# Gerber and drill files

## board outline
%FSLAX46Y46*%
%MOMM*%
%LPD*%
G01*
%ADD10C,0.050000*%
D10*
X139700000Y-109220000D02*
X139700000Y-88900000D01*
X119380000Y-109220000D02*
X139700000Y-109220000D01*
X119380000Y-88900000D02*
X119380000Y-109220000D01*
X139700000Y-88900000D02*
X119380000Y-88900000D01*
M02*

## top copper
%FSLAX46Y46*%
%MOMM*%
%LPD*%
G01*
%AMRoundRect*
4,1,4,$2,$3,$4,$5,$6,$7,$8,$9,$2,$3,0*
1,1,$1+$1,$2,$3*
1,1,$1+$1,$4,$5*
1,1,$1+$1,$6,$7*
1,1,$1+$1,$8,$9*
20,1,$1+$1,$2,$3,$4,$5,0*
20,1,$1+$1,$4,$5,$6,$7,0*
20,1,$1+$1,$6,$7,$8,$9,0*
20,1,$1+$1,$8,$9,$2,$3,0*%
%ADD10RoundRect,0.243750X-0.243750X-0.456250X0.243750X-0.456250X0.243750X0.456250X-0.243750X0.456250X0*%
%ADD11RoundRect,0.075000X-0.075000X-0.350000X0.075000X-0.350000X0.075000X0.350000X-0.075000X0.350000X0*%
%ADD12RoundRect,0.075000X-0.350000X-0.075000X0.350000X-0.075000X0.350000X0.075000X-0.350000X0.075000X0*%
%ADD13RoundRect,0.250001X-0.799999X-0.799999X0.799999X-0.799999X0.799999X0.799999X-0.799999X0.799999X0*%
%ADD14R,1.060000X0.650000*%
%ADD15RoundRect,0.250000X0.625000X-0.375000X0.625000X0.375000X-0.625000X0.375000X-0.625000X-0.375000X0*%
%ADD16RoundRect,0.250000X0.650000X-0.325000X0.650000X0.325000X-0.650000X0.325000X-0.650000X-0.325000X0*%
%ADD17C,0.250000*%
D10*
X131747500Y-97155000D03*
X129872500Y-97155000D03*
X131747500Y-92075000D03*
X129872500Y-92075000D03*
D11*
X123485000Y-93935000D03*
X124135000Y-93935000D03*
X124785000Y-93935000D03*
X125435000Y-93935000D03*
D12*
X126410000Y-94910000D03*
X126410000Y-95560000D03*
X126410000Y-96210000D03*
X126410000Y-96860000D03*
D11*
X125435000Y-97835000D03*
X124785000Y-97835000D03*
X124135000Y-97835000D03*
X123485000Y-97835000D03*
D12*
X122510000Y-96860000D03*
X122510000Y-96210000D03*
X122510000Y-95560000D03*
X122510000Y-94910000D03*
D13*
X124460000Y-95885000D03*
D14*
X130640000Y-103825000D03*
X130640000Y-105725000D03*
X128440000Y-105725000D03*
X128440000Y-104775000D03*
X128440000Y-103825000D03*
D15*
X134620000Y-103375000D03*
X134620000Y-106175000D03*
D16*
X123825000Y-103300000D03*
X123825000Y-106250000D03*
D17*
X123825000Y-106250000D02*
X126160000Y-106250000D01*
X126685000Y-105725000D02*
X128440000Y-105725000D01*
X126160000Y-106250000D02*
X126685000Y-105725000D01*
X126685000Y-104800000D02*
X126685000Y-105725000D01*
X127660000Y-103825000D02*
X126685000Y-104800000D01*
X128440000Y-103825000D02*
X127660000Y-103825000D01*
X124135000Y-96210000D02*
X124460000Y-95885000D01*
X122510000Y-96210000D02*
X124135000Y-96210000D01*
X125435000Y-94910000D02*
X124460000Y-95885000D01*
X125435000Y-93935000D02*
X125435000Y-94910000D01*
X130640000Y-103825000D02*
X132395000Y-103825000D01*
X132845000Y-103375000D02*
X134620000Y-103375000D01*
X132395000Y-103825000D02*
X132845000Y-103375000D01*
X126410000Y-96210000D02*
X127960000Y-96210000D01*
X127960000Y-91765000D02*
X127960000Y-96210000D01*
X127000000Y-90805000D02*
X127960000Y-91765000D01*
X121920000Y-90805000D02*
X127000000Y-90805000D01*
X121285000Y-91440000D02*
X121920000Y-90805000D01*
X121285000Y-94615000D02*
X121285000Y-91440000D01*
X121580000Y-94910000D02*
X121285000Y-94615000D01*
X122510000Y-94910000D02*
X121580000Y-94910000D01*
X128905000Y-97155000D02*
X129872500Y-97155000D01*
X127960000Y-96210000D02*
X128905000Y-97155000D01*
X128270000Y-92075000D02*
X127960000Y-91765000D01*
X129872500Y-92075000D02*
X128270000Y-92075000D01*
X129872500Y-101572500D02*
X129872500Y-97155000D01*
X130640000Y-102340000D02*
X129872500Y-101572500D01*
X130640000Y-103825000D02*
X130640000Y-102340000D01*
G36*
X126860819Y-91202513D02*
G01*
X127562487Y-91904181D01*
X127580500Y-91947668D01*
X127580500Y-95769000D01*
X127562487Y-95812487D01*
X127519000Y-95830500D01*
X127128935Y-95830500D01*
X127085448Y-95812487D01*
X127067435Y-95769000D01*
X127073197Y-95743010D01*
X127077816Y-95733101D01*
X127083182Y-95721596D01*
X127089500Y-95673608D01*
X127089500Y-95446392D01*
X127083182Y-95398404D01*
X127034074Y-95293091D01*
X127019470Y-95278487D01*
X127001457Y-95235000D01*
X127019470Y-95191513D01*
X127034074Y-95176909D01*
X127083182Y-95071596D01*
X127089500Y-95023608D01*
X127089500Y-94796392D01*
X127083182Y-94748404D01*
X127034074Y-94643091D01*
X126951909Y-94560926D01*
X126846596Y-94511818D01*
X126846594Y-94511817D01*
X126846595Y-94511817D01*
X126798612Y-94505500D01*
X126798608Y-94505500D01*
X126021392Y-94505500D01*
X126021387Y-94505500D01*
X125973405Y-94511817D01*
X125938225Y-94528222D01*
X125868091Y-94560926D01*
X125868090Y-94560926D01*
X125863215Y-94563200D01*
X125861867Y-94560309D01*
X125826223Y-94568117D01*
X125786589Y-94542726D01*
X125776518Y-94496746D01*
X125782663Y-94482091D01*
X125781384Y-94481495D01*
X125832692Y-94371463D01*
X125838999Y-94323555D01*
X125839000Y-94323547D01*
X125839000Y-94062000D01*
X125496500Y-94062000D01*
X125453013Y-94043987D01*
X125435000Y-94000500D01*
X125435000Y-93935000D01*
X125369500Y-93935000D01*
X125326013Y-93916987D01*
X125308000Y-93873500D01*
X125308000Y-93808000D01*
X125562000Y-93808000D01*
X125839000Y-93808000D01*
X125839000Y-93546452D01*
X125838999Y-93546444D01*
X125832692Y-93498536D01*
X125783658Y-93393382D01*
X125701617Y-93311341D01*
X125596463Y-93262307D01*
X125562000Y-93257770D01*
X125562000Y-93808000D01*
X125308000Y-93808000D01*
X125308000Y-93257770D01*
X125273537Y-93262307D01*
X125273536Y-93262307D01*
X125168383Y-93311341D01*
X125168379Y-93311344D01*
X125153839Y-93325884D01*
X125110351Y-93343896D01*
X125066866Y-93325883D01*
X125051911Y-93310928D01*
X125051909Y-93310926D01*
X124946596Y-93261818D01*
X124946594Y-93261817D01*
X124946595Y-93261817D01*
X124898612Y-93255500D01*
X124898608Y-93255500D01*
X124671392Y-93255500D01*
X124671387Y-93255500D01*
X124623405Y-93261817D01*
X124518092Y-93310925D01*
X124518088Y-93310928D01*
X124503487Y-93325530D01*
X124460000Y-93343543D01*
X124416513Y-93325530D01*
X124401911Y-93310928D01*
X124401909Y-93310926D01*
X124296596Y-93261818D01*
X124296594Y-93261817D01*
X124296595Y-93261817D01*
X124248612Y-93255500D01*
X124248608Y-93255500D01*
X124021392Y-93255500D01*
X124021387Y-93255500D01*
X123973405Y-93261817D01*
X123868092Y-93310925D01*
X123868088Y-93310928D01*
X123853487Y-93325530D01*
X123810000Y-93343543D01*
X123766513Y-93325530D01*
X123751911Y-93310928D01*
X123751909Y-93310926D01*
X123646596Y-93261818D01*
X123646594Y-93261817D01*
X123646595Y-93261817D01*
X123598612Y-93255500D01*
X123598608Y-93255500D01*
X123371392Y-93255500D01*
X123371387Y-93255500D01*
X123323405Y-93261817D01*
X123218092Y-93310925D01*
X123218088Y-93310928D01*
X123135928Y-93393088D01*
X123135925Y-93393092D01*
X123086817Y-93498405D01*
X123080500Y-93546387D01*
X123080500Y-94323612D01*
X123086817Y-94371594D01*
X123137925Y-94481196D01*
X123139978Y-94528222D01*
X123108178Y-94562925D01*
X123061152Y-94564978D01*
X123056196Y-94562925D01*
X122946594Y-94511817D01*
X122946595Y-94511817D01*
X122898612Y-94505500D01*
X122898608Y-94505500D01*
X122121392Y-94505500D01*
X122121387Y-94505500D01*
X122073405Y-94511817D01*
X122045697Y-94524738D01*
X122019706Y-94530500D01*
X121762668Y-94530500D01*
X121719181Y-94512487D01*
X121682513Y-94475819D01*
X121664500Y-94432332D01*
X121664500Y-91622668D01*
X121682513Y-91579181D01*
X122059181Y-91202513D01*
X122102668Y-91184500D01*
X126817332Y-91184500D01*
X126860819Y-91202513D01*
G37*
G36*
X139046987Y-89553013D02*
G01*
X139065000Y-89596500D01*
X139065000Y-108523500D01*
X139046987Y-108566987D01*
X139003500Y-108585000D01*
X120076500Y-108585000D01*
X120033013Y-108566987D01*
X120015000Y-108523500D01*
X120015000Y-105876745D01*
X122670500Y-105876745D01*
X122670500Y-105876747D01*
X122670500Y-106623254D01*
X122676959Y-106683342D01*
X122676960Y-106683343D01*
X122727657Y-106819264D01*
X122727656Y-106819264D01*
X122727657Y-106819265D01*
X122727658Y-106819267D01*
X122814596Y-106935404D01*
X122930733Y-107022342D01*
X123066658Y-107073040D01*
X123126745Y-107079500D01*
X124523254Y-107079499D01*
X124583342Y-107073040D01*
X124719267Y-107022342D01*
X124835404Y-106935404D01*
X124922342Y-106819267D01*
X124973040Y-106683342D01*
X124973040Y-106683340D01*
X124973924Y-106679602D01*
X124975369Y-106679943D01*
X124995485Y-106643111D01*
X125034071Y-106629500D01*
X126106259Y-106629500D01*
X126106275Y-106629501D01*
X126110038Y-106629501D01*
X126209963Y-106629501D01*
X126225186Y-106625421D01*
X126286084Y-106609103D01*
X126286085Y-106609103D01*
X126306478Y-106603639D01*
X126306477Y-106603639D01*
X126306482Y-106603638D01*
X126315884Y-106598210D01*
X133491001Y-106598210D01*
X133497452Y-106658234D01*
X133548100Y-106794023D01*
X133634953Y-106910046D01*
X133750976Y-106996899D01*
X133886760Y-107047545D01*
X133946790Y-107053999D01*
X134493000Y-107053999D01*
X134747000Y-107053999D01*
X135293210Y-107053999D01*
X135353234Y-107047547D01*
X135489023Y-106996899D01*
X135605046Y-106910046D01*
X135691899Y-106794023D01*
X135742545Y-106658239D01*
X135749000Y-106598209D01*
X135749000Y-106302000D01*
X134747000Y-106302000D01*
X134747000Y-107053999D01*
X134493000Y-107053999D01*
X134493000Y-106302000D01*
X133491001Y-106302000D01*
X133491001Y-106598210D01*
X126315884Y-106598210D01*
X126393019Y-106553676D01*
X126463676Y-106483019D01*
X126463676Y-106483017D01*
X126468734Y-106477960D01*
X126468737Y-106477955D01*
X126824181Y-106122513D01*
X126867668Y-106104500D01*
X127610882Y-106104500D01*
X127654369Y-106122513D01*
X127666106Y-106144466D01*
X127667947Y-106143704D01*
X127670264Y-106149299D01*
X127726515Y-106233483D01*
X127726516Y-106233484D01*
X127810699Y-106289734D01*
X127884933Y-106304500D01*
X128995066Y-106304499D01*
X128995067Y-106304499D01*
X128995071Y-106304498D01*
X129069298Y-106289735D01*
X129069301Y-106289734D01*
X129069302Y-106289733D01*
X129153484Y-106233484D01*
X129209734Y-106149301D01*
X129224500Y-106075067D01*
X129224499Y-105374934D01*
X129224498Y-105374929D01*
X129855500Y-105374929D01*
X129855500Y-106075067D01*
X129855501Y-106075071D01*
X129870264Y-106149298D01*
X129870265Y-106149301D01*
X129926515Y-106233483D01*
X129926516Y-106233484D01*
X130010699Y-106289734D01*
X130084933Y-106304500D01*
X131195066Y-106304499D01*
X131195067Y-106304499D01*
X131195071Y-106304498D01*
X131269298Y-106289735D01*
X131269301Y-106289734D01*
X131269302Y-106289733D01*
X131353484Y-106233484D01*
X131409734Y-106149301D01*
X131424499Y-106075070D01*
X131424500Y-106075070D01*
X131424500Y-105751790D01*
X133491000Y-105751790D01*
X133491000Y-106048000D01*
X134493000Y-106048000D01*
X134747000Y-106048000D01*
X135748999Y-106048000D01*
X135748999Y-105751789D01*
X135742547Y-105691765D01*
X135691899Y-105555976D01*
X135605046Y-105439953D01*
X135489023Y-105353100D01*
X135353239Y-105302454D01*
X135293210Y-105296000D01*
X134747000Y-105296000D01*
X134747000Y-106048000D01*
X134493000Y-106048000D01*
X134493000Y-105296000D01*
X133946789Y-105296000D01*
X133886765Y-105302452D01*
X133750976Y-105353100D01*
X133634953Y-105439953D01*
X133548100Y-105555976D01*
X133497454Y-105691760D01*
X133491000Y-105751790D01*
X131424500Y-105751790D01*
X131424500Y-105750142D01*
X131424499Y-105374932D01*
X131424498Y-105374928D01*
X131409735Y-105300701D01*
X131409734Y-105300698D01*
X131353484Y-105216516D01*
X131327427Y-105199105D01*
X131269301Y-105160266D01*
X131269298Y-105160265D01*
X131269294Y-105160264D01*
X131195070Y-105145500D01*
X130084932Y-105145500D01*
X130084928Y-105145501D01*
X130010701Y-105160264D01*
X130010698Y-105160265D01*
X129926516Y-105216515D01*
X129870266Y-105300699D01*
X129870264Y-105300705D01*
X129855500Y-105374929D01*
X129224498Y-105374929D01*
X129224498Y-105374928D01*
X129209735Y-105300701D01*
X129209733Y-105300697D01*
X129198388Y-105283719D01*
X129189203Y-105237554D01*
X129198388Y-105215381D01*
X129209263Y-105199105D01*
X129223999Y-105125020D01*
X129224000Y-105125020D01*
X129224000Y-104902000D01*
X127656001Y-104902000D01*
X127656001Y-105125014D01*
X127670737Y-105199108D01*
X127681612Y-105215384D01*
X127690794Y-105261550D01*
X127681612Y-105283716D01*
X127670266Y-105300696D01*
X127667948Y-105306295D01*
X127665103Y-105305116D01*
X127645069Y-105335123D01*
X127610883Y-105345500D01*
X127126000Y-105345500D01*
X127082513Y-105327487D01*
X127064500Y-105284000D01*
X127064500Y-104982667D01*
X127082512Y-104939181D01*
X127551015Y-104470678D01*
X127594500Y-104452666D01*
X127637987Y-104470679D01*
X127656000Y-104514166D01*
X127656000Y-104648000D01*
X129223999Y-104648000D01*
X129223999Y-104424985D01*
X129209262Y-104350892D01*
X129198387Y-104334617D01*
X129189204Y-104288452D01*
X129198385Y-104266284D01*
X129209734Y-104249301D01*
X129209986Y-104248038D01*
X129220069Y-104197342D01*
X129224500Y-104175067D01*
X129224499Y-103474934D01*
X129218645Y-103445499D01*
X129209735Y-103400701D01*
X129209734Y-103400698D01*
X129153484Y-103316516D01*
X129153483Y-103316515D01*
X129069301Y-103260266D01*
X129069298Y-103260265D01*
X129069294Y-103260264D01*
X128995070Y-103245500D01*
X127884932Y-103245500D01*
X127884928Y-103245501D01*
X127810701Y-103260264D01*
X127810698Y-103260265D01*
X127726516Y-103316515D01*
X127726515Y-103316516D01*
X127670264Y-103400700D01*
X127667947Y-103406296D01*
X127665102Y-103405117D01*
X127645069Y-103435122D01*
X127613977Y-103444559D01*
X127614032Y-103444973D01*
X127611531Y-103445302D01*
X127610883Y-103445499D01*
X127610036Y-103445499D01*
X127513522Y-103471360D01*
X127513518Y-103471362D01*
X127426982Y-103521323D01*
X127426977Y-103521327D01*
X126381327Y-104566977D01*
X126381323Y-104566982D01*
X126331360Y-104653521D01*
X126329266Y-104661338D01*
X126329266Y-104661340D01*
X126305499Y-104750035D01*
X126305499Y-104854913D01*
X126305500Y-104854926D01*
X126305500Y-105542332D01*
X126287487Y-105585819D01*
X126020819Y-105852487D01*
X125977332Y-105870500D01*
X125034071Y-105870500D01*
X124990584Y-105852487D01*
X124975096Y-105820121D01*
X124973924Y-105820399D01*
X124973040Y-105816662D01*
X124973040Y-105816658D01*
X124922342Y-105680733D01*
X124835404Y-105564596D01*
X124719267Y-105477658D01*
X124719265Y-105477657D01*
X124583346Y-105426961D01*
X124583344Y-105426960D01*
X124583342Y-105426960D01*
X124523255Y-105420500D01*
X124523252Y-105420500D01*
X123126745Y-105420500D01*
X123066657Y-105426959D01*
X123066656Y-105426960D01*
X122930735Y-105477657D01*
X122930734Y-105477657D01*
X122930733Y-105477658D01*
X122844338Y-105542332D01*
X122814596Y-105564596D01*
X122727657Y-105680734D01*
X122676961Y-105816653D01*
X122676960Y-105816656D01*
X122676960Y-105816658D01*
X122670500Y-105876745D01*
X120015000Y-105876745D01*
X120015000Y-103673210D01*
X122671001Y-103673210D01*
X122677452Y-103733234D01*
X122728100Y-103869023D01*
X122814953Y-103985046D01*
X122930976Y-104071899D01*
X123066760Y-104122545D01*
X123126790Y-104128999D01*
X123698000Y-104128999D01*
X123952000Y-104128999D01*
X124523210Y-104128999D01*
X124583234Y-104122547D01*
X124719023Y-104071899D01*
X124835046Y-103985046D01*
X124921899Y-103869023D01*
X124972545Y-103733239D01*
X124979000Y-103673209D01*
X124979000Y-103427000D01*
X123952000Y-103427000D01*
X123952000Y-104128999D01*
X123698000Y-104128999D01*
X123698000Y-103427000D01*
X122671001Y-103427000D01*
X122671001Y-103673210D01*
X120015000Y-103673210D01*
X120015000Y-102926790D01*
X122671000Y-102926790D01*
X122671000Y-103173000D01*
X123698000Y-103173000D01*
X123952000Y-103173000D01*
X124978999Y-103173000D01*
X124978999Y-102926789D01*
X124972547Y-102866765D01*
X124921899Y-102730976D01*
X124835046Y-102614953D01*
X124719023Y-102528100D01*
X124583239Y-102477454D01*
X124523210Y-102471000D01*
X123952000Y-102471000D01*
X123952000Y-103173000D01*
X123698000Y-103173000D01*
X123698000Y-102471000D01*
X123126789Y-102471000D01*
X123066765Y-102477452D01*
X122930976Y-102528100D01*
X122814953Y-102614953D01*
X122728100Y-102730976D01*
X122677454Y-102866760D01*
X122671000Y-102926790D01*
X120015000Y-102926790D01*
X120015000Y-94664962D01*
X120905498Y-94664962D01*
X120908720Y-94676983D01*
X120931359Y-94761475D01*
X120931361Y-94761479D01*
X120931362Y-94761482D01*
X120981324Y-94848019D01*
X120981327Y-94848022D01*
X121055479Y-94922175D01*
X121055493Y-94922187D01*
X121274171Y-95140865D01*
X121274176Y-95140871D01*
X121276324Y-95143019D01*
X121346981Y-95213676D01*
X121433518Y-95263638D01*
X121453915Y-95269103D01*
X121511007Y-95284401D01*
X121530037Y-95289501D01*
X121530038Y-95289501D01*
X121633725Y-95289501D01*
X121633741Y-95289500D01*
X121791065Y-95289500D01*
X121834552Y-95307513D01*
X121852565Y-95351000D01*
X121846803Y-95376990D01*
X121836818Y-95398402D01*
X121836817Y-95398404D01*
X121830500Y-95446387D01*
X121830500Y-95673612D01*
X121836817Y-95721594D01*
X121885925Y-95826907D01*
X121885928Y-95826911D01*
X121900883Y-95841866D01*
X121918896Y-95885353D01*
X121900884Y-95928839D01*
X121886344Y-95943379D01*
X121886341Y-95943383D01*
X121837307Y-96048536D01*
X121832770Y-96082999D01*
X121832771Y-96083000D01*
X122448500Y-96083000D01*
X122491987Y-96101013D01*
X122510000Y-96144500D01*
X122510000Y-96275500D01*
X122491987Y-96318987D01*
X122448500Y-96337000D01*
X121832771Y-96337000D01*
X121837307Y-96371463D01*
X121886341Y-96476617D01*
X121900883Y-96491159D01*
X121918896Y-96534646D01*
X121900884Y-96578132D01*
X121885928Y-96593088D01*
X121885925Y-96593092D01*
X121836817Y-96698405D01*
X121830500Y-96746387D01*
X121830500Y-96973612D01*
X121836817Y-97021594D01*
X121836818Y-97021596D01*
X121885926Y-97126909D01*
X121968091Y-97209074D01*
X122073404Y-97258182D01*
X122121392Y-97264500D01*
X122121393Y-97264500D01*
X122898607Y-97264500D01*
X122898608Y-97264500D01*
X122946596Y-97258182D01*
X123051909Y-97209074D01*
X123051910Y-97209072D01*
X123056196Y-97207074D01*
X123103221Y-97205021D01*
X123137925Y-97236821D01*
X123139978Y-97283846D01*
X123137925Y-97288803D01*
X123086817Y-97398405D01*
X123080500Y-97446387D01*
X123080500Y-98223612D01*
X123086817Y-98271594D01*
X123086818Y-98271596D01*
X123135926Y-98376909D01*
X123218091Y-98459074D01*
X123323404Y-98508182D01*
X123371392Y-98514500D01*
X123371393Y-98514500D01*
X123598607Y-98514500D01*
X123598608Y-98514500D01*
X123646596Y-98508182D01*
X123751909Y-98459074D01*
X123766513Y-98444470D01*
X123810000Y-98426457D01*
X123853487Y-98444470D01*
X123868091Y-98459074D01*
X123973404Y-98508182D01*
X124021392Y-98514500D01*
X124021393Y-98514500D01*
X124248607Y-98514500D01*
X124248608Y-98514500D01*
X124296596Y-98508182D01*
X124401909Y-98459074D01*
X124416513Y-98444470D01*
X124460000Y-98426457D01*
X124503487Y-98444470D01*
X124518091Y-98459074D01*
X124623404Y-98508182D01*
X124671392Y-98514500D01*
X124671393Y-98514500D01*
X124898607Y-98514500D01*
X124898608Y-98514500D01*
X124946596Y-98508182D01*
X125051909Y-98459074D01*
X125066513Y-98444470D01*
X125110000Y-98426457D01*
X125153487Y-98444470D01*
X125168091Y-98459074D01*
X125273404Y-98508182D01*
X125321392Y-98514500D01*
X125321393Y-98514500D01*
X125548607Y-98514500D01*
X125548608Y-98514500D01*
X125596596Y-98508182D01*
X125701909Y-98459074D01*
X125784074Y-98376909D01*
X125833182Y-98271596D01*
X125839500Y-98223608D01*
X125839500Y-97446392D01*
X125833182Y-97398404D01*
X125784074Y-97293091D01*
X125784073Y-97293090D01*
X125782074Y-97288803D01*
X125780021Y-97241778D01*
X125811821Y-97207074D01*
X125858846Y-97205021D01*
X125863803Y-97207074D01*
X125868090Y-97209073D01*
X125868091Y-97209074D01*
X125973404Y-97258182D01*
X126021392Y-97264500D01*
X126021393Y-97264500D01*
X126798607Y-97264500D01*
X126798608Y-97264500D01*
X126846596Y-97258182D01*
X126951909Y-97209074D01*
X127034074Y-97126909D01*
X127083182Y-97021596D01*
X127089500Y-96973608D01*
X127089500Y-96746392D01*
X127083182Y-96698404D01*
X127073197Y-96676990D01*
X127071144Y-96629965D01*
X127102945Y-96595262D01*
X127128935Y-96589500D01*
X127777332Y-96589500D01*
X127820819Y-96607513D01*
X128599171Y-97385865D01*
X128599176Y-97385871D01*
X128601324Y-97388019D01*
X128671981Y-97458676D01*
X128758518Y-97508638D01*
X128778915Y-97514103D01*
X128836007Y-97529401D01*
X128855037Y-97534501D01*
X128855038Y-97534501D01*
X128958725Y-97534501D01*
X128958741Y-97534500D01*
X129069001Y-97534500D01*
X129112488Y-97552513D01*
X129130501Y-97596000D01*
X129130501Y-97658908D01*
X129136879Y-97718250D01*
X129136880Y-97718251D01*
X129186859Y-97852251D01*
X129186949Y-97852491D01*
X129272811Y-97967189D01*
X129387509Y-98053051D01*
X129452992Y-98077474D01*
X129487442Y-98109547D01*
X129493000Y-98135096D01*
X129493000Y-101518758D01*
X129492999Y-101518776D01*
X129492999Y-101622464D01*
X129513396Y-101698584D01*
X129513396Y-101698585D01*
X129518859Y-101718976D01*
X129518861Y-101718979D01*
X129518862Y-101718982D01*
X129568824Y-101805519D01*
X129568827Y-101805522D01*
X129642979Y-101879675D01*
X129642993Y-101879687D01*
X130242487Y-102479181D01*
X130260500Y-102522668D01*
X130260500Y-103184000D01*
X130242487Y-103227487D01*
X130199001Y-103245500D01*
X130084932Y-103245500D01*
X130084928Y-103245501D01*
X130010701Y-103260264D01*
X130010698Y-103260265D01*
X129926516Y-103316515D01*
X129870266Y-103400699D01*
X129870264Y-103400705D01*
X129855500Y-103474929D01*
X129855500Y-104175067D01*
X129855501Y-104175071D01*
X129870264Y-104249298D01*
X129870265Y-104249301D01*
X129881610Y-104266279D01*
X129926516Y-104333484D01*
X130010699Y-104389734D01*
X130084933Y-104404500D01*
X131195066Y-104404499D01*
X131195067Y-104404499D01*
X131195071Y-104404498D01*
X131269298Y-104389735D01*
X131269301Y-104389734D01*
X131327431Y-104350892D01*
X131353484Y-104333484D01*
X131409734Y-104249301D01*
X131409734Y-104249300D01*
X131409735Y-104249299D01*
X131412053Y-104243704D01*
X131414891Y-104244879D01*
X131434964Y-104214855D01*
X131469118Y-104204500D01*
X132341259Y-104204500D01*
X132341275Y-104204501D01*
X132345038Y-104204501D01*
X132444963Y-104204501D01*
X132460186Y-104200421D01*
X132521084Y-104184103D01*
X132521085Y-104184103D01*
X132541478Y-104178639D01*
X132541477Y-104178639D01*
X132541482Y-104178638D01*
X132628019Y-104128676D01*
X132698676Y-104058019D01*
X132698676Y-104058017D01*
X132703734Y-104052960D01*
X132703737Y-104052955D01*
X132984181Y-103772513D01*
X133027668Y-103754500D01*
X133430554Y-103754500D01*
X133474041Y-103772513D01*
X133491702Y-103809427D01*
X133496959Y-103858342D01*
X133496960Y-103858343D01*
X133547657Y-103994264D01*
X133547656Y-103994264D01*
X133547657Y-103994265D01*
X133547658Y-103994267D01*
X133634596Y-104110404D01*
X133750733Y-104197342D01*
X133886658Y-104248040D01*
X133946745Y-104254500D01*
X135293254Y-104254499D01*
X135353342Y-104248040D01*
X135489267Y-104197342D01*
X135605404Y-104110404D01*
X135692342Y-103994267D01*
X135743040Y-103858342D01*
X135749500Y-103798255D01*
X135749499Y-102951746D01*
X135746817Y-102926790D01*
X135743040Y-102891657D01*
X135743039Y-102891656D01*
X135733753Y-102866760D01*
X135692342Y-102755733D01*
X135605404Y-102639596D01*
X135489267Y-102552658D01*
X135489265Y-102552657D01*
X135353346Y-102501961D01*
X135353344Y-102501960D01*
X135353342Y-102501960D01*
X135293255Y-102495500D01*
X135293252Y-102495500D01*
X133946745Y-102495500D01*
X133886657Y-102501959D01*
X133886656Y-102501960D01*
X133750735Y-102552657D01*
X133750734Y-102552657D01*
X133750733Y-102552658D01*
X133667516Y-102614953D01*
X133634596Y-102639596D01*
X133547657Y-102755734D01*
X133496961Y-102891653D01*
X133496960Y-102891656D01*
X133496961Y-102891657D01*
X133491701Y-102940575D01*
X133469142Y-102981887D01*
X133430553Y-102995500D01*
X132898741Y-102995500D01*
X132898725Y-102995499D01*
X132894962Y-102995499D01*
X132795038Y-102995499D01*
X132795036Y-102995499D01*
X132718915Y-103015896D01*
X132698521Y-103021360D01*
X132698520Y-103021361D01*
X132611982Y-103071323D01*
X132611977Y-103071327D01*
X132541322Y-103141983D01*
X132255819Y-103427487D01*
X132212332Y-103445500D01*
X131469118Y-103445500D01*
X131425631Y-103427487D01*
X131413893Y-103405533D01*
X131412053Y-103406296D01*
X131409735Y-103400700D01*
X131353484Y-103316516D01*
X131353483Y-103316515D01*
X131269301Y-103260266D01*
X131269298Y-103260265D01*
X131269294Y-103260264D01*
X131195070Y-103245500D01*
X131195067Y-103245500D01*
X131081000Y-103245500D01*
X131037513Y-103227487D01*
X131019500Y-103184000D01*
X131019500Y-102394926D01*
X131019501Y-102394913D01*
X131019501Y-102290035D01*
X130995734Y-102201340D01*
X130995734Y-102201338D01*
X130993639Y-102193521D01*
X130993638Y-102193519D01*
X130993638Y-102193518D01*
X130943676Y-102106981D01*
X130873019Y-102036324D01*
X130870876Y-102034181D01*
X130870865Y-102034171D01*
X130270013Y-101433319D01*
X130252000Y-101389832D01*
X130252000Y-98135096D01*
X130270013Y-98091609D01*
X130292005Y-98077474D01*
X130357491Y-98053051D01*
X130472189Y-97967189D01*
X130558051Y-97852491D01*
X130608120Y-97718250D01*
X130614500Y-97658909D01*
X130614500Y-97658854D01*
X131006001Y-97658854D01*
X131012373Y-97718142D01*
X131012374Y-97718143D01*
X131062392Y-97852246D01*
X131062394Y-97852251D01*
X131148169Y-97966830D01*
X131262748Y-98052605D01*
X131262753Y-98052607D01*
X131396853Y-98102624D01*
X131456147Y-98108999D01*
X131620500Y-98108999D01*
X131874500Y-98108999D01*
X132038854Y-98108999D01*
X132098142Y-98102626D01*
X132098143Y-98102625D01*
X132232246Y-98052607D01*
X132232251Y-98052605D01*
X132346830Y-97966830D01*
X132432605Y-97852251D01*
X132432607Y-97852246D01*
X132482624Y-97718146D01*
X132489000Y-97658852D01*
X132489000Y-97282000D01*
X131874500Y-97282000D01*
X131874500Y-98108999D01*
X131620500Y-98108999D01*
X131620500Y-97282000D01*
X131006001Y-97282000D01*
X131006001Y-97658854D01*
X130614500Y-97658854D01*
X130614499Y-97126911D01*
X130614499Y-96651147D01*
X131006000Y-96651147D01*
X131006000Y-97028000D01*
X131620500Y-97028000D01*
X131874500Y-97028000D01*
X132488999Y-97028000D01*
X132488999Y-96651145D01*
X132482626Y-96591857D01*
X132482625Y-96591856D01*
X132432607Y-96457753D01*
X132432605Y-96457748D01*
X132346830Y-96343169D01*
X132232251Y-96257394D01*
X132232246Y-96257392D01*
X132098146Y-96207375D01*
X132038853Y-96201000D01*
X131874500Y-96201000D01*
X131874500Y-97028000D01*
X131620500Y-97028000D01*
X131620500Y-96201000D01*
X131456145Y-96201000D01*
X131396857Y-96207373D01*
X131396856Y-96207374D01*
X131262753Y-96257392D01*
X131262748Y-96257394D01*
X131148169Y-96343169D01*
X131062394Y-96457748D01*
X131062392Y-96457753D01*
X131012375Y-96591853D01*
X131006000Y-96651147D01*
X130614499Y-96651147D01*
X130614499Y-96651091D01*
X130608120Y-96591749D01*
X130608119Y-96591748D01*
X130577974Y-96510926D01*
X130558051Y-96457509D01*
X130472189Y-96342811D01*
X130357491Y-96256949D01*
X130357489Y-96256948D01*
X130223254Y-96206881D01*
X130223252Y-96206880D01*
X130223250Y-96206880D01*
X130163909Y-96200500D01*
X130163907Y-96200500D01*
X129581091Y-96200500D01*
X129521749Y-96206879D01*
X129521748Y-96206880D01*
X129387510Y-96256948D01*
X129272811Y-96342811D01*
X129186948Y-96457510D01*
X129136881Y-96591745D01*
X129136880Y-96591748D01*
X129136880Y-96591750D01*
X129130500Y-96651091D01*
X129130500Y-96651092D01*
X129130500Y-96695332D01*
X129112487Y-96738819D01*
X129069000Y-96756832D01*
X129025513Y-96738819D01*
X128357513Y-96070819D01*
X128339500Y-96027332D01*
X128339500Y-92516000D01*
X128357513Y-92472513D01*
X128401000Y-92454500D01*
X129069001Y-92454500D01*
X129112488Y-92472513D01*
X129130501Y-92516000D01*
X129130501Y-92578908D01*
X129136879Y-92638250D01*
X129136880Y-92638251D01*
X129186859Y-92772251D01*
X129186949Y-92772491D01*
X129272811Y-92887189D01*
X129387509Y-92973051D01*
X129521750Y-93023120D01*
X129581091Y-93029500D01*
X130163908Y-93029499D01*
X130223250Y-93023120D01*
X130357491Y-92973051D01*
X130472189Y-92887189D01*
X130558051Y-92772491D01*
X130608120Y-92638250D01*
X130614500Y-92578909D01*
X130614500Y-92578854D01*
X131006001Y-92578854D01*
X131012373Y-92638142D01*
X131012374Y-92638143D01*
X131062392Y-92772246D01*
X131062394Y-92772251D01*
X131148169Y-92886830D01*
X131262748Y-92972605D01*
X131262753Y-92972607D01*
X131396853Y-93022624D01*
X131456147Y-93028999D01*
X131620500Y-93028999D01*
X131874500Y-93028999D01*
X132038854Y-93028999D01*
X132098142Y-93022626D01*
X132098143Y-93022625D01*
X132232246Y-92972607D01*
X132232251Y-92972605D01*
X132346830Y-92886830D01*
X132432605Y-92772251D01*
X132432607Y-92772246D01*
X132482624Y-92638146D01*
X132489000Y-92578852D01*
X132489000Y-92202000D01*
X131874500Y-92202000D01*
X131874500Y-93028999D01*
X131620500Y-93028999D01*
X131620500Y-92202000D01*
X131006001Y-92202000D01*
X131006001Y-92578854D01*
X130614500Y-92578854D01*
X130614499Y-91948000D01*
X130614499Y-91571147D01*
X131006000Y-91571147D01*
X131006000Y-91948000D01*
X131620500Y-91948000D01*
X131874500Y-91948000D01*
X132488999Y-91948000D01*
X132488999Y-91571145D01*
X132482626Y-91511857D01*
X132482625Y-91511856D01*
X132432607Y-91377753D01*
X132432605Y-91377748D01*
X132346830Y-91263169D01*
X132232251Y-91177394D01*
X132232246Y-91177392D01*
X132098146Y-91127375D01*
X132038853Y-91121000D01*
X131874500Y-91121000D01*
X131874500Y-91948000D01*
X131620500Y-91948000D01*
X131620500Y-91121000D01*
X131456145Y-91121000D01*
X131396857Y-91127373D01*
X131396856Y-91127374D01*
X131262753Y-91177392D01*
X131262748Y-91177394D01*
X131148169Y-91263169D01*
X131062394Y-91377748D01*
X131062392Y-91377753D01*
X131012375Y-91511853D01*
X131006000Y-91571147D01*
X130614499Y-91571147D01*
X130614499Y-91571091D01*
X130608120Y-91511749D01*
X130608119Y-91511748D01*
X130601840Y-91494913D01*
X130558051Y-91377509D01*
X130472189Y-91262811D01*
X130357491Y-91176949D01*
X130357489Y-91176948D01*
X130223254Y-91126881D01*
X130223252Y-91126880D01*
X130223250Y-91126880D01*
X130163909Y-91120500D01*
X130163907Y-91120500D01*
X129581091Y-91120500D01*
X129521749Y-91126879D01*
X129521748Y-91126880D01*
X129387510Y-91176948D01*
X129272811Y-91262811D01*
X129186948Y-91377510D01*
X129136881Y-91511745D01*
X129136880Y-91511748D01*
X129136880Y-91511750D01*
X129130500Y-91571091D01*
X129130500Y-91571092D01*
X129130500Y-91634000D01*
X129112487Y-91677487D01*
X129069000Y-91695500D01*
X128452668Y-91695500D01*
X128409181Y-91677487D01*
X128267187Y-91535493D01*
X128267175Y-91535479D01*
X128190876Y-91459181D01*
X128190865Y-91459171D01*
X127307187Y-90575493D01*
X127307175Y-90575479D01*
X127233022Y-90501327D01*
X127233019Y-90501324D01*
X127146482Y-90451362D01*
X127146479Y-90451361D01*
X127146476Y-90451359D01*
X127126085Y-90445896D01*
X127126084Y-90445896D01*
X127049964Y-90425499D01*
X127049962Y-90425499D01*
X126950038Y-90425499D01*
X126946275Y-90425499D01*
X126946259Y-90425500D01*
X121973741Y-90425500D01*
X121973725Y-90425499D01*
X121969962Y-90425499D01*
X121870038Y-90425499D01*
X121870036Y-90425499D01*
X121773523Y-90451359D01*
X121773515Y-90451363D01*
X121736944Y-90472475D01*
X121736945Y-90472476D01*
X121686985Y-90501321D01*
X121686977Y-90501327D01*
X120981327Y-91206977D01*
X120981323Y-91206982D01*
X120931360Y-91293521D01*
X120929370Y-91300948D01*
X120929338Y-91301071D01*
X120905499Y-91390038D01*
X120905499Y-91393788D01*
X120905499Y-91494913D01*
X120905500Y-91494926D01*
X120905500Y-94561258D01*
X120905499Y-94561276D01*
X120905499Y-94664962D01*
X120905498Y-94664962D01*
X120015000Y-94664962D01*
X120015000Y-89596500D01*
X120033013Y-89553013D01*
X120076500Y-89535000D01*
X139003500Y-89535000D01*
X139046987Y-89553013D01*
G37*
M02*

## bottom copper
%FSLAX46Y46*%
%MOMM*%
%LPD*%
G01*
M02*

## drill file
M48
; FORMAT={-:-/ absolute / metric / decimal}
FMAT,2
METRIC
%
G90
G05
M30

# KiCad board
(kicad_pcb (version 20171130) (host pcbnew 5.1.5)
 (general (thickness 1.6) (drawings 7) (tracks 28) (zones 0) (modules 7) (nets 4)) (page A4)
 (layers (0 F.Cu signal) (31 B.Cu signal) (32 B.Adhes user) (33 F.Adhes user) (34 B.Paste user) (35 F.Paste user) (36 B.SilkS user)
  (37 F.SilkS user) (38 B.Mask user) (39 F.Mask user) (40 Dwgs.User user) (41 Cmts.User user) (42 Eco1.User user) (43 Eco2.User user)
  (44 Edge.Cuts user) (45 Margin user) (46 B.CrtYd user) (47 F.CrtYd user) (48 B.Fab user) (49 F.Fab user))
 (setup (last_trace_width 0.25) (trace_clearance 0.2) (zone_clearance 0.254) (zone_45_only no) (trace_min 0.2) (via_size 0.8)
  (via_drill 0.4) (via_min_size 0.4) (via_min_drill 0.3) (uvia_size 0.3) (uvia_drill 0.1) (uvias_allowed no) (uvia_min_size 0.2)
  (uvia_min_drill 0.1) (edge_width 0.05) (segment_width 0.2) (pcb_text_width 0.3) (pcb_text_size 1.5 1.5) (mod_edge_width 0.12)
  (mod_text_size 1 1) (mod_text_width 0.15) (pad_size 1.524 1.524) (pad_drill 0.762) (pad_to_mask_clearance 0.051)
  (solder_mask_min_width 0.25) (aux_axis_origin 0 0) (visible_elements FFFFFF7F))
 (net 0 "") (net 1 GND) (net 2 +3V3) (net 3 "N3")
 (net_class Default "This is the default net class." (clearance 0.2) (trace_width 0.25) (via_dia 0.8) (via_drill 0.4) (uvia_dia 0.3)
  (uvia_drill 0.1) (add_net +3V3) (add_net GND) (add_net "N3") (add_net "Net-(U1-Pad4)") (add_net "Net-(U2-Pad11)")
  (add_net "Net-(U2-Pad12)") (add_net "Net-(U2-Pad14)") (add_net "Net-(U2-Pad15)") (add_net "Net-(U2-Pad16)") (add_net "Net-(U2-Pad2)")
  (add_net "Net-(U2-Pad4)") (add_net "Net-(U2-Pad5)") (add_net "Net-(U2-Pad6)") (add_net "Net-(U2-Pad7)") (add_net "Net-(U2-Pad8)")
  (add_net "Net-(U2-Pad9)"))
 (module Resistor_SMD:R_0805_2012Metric (layer F.Cu) (at 130.81 97.155)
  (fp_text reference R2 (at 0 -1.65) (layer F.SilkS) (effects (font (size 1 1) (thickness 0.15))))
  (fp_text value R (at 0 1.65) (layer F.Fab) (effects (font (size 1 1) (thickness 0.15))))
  (pad 2 smd roundrect (at 0.9375 0) (size 0.975 1.4) (layers F.Cu F.Paste F.Mask) (roundrect_rratio 0.25) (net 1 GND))
  (pad 1 smd roundrect (at -0.9375 0) (size 0.975 1.4) (layers F.Cu F.Paste F.Mask) (roundrect_rratio 0.25) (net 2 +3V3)))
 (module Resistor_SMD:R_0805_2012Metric (layer F.Cu) (at 130.81 92.075)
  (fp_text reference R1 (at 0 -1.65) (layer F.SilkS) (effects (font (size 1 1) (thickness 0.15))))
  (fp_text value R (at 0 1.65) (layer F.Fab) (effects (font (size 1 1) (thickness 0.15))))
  (pad 2 smd roundrect (at 0.9375 0) (size 0.975 1.4) (layers F.Cu F.Paste F.Mask) (roundrect_rratio 0.25) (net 1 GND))
  (pad 1 smd roundrect (at -0.9375 0) (size 0.975 1.4) (layers F.Cu F.Paste F.Mask) (roundrect_rratio 0.25) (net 2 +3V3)))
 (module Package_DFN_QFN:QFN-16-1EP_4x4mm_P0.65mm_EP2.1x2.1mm (layer F.Cu) (at 124.46 95.885)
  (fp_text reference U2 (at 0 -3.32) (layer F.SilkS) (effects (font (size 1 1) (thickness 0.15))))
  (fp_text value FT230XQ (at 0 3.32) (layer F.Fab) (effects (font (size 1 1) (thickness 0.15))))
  (pad 16 smd roundrect (at -0.975 -1.95) (size 0.3 0.85) (layers F.Cu F.Paste F.Mask) (roundrect_rratio 0.25))
  (pad 15 smd roundrect (at -0.325 -1.95) (size 0.3 0.85) (layers F.Cu F.Paste F.Mask) (roundrect_rratio 0.25))
  (pad 14 smd roundrect (at 0.325 -1.95) (size 0.3 0.85) (layers F.Cu F.Paste F.Mask) (roundrect_rratio 0.25))
  (pad 13 smd roundrect (at 0.975 -1.95) (size 0.3 0.85) (layers F.Cu F.Paste F.Mask) (roundrect_rratio 0.25) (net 1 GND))
  (pad 12 smd roundrect (at 1.95 -0.975) (size 0.85 0.3) (layers F.Cu F.Paste F.Mask) (roundrect_rratio 0.25))
  (pad 11 smd roundrect (at 1.95 -0.325) (size 0.85 0.3) (layers F.Cu F.Paste F.Mask) (roundrect_rratio 0.25))
  (pad 10 smd roundrect (at 1.95 0.325) (size 0.85 0.3) (layers F.Cu F.Paste F.Mask) (roundrect_rratio 0.25) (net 2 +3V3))
  (pad 9 smd roundrect (at 1.95 0.975) (size 0.85 0.3) (layers F.Cu F.Paste F.Mask) (roundrect_rratio 0.25))
  (pad 8 smd roundrect (at 0.975 1.95) (size 0.3 0.85) (layers F.Cu F.Paste F.Mask) (roundrect_rratio 0.25))
  (pad 7 smd roundrect (at 0.325 1.95) (size 0.3 0.85) (layers F.Cu F.Paste F.Mask) (roundrect_rratio 0.25))
  (pad 6 smd roundrect (at -0.325 1.95) (size 0.3 0.85) (layers F.Cu F.Paste F.Mask) (roundrect_rratio 0.25))
  (pad 5 smd roundrect (at -0.975 1.95) (size 0.3 0.85) (layers F.Cu F.Paste F.Mask) (roundrect_rratio 0.25))
  (pad 4 smd roundrect (at -1.95 0.975) (size 0.85 0.3) (layers F.Cu F.Paste F.Mask) (roundrect_rratio 0.25))
  (pad 3 smd roundrect (at -1.95 0.325) (size 0.85 0.3) (layers F.Cu F.Paste F.Mask) (roundrect_rratio 0.25) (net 1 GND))
  (pad 2 smd roundrect (at -1.95 -0.325) (size 0.85 0.3) (layers F.Cu F.Paste F.Mask) (roundrect_rratio 0.25))
  (pad 1 smd roundrect (at -1.95 -0.975) (size 0.85 0.3) (layers F.Cu F.Paste F.Mask) (roundrect_rratio 0.25) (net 2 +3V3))
  (pad "" smd roundrect (at 0.525 0.525) (size 0.85 0.85) (layers F.Paste) (roundrect_rratio 0.25))
  (pad "" smd roundrect (at 0.525 -0.525) (size 0.85 0.85) (layers F.Paste) (roundrect_rratio 0.25))
  (pad "" smd roundrect (at -0.525 0.525) (size 0.85 0.85) (layers F.Paste) (roundrect_rratio 0.25))
  (pad "" smd roundrect (at -0.525 -0.525) (size 0.85 0.85) (layers F.Paste) (roundrect_rratio 0.25))
  (pad 17 smd roundrect (at 0 0) (size 2.1 2.1) (layers F.Cu F.Mask) (roundrect_rratio 0.119048) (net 1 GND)))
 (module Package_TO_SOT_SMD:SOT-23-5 (layer F.Cu) (at 129.54 104.775)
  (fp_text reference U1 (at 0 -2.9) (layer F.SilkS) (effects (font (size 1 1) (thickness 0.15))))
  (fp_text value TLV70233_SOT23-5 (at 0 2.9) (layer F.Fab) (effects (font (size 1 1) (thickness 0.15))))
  (pad 5 smd rect (at 1.1 -0.95) (size 1.06 0.65) (layers F.Cu F.Paste F.Mask) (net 2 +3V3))
  (pad 4 smd rect (at 1.1 0.95) (size 1.06 0.65) (layers F.Cu F.Paste F.Mask))
  (pad 3 smd rect (at -1.1 0.95) (size 1.06 0.65) (layers F.Cu F.Paste F.Mask) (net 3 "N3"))
  (pad 2 smd rect (at -1.1 0) (size 1.06 0.65) (layers F.Cu F.Paste F.Mask) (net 1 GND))
  (pad 1 smd rect (at -1.1 -0.95) (size 1.06 0.65) (layers F.Cu F.Paste F.Mask) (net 3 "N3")))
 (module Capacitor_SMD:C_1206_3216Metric (layer F.Cu) (at 134.62 104.775 90)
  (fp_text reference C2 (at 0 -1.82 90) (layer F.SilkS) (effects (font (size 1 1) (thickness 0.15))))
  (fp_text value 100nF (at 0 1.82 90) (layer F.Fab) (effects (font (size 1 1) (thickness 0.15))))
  (pad 2 smd roundrect (at 1.4 0 90) (size 1.25 1.75) (layers F.Cu F.Paste F.Mask) (roundrect_rratio 0.2) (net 2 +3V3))
  (pad 1 smd roundrect (at -1.4 0 90) (size 1.25 1.75) (layers F.Cu F.Paste F.Mask) (roundrect_rratio 0.2) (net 1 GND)))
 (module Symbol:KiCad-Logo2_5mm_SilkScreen (layer F.Cu) (at 135.89 95.885 90)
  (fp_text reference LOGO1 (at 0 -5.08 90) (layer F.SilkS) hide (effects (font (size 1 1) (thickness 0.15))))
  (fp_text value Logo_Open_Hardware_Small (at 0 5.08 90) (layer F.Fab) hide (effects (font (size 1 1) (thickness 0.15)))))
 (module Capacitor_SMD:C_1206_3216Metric (layer F.Cu) (at 123.825 104.775 90)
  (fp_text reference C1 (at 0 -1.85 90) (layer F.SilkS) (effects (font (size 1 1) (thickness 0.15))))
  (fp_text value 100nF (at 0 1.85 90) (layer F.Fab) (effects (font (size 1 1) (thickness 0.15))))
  (pad 2 smd roundrect (at 1.475 0 90) (size 1.15 1.8) (layers F.Cu F.Paste F.Mask) (roundrect_rratio 0.217391) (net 1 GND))
  (pad 1 smd roundrect (at -1.475 0 90) (size 1.15 1.8) (layers F.Cu F.Paste F.Mask) (roundrect_rratio 0.217391) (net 3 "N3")))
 (gr_line (start 139.7 109.22) (end 139.7 88.9) (layer Edge.Cuts) (width 0.05))
 (gr_line (start 119.38 109.22) (end 139.7 109.22) (layer Edge.Cuts) (width 0.05))
 (gr_line (start 119.38 88.9) (end 119.38 109.22) (layer Edge.Cuts) (width 0.05))
 (gr_line (start 139.7 88.9) (end 119.38 88.9) (layer Edge.Cuts) (width 0.05))
 (segment (start 123.825 106.25) (end 126.16 106.25) (width 0.25) (layer F.Cu) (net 3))
 (segment (start 126.685 105.725) (end 128.44 105.725) (width 0.25) (layer F.Cu) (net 3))
 (segment (start 126.16 106.25) (end 126.685 105.725) (width 0.25) (layer F.Cu) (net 3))
 (segment (start 126.685 104.8) (end 126.685 105.725) (width 0.25) (layer F.Cu) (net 3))
 (segment (start 127.66 103.825) (end 126.685 104.8) (width 0.25) (layer F.Cu) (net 3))
 (segment (start 128.44 103.825) (end 127.66 103.825) (width 0.25) (layer F.Cu) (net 3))
 (segment (start 124.135 96.21) (end 124.46 95.885) (width 0.25) (layer F.Cu) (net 1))
 (segment (start 122.51 96.21) (end 124.135 96.21) (width 0.25) (layer F.Cu) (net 1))
 (segment (start 125.435 94.91) (end 124.46 95.885) (width 0.25) (layer F.Cu) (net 1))
 (segment (start 125.435 93.935) (end 125.435 94.91) (width 0.25) (layer F.Cu) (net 1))
 (segment (start 130.64 103.825) (end 132.395 103.825) (width 0.25) (layer F.Cu) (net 2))
 (segment (start 132.845 103.375) (end 134.62 103.375) (width 0.25) (layer F.Cu) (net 2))
 (segment (start 132.395 103.825) (end 132.845 103.375) (width 0.25) (layer F.Cu) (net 2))
 (segment (start 126.41 96.21) (end 127.96 96.21) (width 0.25) (layer F.Cu) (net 2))
 (segment (start 127.96 91.765) (end 127.96 96.21) (width 0.25) (layer F.Cu) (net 2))
 (segment (start 127 90.805) (end 127.96 91.765) (width 0.25) (layer F.Cu) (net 2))
 (segment (start 121.92 90.805) (end 127 90.805) (width 0.25) (layer F.Cu) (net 2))
 (segment (start 121.285 91.44) (end 121.92 90.805) (width 0.25) (layer F.Cu) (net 2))
 (segment (start 121.285 94.615) (end 121.285 91.44) (width 0.25) (layer F.Cu) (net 2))
 (segment (start 121.58 94.91) (end 121.285 94.615) (width 0.25) (layer F.Cu) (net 2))
 (segment (start 122.51 94.91) (end 121.58 94.91) (width 0.25) (layer F.Cu) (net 2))
 (segment (start 128.905 97.155) (end 129.8725 97.155) (width 0.25) (layer F.Cu) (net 2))
 (segment (start 127.96 96.21) (end 128.905 97.155) (width 0.25) (layer F.Cu) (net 2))
 (segment (start 128.27 92.075) (end 127.96 91.765) (width 0.25) (layer F.Cu) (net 2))
 (segment (start 129.8725 92.075) (end 128.27 92.075) (width 0.25) (layer F.Cu) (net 2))
 (segment (start 129.8725 101.5725) (end 129.8725 97.155) (width 0.25) (layer F.Cu) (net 2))
 (segment (start 130.64 102.34) (end 129.8725 101.5725) (width 0.25) (layer F.Cu) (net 2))
 (segment (start 130.64 103.825) (end 130.64 102.34) (width 0.25) (layer F.Cu) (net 2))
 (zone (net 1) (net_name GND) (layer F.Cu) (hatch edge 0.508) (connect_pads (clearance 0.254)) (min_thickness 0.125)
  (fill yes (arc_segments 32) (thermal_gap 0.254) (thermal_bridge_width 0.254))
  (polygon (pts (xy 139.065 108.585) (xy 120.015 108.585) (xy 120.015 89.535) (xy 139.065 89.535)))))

